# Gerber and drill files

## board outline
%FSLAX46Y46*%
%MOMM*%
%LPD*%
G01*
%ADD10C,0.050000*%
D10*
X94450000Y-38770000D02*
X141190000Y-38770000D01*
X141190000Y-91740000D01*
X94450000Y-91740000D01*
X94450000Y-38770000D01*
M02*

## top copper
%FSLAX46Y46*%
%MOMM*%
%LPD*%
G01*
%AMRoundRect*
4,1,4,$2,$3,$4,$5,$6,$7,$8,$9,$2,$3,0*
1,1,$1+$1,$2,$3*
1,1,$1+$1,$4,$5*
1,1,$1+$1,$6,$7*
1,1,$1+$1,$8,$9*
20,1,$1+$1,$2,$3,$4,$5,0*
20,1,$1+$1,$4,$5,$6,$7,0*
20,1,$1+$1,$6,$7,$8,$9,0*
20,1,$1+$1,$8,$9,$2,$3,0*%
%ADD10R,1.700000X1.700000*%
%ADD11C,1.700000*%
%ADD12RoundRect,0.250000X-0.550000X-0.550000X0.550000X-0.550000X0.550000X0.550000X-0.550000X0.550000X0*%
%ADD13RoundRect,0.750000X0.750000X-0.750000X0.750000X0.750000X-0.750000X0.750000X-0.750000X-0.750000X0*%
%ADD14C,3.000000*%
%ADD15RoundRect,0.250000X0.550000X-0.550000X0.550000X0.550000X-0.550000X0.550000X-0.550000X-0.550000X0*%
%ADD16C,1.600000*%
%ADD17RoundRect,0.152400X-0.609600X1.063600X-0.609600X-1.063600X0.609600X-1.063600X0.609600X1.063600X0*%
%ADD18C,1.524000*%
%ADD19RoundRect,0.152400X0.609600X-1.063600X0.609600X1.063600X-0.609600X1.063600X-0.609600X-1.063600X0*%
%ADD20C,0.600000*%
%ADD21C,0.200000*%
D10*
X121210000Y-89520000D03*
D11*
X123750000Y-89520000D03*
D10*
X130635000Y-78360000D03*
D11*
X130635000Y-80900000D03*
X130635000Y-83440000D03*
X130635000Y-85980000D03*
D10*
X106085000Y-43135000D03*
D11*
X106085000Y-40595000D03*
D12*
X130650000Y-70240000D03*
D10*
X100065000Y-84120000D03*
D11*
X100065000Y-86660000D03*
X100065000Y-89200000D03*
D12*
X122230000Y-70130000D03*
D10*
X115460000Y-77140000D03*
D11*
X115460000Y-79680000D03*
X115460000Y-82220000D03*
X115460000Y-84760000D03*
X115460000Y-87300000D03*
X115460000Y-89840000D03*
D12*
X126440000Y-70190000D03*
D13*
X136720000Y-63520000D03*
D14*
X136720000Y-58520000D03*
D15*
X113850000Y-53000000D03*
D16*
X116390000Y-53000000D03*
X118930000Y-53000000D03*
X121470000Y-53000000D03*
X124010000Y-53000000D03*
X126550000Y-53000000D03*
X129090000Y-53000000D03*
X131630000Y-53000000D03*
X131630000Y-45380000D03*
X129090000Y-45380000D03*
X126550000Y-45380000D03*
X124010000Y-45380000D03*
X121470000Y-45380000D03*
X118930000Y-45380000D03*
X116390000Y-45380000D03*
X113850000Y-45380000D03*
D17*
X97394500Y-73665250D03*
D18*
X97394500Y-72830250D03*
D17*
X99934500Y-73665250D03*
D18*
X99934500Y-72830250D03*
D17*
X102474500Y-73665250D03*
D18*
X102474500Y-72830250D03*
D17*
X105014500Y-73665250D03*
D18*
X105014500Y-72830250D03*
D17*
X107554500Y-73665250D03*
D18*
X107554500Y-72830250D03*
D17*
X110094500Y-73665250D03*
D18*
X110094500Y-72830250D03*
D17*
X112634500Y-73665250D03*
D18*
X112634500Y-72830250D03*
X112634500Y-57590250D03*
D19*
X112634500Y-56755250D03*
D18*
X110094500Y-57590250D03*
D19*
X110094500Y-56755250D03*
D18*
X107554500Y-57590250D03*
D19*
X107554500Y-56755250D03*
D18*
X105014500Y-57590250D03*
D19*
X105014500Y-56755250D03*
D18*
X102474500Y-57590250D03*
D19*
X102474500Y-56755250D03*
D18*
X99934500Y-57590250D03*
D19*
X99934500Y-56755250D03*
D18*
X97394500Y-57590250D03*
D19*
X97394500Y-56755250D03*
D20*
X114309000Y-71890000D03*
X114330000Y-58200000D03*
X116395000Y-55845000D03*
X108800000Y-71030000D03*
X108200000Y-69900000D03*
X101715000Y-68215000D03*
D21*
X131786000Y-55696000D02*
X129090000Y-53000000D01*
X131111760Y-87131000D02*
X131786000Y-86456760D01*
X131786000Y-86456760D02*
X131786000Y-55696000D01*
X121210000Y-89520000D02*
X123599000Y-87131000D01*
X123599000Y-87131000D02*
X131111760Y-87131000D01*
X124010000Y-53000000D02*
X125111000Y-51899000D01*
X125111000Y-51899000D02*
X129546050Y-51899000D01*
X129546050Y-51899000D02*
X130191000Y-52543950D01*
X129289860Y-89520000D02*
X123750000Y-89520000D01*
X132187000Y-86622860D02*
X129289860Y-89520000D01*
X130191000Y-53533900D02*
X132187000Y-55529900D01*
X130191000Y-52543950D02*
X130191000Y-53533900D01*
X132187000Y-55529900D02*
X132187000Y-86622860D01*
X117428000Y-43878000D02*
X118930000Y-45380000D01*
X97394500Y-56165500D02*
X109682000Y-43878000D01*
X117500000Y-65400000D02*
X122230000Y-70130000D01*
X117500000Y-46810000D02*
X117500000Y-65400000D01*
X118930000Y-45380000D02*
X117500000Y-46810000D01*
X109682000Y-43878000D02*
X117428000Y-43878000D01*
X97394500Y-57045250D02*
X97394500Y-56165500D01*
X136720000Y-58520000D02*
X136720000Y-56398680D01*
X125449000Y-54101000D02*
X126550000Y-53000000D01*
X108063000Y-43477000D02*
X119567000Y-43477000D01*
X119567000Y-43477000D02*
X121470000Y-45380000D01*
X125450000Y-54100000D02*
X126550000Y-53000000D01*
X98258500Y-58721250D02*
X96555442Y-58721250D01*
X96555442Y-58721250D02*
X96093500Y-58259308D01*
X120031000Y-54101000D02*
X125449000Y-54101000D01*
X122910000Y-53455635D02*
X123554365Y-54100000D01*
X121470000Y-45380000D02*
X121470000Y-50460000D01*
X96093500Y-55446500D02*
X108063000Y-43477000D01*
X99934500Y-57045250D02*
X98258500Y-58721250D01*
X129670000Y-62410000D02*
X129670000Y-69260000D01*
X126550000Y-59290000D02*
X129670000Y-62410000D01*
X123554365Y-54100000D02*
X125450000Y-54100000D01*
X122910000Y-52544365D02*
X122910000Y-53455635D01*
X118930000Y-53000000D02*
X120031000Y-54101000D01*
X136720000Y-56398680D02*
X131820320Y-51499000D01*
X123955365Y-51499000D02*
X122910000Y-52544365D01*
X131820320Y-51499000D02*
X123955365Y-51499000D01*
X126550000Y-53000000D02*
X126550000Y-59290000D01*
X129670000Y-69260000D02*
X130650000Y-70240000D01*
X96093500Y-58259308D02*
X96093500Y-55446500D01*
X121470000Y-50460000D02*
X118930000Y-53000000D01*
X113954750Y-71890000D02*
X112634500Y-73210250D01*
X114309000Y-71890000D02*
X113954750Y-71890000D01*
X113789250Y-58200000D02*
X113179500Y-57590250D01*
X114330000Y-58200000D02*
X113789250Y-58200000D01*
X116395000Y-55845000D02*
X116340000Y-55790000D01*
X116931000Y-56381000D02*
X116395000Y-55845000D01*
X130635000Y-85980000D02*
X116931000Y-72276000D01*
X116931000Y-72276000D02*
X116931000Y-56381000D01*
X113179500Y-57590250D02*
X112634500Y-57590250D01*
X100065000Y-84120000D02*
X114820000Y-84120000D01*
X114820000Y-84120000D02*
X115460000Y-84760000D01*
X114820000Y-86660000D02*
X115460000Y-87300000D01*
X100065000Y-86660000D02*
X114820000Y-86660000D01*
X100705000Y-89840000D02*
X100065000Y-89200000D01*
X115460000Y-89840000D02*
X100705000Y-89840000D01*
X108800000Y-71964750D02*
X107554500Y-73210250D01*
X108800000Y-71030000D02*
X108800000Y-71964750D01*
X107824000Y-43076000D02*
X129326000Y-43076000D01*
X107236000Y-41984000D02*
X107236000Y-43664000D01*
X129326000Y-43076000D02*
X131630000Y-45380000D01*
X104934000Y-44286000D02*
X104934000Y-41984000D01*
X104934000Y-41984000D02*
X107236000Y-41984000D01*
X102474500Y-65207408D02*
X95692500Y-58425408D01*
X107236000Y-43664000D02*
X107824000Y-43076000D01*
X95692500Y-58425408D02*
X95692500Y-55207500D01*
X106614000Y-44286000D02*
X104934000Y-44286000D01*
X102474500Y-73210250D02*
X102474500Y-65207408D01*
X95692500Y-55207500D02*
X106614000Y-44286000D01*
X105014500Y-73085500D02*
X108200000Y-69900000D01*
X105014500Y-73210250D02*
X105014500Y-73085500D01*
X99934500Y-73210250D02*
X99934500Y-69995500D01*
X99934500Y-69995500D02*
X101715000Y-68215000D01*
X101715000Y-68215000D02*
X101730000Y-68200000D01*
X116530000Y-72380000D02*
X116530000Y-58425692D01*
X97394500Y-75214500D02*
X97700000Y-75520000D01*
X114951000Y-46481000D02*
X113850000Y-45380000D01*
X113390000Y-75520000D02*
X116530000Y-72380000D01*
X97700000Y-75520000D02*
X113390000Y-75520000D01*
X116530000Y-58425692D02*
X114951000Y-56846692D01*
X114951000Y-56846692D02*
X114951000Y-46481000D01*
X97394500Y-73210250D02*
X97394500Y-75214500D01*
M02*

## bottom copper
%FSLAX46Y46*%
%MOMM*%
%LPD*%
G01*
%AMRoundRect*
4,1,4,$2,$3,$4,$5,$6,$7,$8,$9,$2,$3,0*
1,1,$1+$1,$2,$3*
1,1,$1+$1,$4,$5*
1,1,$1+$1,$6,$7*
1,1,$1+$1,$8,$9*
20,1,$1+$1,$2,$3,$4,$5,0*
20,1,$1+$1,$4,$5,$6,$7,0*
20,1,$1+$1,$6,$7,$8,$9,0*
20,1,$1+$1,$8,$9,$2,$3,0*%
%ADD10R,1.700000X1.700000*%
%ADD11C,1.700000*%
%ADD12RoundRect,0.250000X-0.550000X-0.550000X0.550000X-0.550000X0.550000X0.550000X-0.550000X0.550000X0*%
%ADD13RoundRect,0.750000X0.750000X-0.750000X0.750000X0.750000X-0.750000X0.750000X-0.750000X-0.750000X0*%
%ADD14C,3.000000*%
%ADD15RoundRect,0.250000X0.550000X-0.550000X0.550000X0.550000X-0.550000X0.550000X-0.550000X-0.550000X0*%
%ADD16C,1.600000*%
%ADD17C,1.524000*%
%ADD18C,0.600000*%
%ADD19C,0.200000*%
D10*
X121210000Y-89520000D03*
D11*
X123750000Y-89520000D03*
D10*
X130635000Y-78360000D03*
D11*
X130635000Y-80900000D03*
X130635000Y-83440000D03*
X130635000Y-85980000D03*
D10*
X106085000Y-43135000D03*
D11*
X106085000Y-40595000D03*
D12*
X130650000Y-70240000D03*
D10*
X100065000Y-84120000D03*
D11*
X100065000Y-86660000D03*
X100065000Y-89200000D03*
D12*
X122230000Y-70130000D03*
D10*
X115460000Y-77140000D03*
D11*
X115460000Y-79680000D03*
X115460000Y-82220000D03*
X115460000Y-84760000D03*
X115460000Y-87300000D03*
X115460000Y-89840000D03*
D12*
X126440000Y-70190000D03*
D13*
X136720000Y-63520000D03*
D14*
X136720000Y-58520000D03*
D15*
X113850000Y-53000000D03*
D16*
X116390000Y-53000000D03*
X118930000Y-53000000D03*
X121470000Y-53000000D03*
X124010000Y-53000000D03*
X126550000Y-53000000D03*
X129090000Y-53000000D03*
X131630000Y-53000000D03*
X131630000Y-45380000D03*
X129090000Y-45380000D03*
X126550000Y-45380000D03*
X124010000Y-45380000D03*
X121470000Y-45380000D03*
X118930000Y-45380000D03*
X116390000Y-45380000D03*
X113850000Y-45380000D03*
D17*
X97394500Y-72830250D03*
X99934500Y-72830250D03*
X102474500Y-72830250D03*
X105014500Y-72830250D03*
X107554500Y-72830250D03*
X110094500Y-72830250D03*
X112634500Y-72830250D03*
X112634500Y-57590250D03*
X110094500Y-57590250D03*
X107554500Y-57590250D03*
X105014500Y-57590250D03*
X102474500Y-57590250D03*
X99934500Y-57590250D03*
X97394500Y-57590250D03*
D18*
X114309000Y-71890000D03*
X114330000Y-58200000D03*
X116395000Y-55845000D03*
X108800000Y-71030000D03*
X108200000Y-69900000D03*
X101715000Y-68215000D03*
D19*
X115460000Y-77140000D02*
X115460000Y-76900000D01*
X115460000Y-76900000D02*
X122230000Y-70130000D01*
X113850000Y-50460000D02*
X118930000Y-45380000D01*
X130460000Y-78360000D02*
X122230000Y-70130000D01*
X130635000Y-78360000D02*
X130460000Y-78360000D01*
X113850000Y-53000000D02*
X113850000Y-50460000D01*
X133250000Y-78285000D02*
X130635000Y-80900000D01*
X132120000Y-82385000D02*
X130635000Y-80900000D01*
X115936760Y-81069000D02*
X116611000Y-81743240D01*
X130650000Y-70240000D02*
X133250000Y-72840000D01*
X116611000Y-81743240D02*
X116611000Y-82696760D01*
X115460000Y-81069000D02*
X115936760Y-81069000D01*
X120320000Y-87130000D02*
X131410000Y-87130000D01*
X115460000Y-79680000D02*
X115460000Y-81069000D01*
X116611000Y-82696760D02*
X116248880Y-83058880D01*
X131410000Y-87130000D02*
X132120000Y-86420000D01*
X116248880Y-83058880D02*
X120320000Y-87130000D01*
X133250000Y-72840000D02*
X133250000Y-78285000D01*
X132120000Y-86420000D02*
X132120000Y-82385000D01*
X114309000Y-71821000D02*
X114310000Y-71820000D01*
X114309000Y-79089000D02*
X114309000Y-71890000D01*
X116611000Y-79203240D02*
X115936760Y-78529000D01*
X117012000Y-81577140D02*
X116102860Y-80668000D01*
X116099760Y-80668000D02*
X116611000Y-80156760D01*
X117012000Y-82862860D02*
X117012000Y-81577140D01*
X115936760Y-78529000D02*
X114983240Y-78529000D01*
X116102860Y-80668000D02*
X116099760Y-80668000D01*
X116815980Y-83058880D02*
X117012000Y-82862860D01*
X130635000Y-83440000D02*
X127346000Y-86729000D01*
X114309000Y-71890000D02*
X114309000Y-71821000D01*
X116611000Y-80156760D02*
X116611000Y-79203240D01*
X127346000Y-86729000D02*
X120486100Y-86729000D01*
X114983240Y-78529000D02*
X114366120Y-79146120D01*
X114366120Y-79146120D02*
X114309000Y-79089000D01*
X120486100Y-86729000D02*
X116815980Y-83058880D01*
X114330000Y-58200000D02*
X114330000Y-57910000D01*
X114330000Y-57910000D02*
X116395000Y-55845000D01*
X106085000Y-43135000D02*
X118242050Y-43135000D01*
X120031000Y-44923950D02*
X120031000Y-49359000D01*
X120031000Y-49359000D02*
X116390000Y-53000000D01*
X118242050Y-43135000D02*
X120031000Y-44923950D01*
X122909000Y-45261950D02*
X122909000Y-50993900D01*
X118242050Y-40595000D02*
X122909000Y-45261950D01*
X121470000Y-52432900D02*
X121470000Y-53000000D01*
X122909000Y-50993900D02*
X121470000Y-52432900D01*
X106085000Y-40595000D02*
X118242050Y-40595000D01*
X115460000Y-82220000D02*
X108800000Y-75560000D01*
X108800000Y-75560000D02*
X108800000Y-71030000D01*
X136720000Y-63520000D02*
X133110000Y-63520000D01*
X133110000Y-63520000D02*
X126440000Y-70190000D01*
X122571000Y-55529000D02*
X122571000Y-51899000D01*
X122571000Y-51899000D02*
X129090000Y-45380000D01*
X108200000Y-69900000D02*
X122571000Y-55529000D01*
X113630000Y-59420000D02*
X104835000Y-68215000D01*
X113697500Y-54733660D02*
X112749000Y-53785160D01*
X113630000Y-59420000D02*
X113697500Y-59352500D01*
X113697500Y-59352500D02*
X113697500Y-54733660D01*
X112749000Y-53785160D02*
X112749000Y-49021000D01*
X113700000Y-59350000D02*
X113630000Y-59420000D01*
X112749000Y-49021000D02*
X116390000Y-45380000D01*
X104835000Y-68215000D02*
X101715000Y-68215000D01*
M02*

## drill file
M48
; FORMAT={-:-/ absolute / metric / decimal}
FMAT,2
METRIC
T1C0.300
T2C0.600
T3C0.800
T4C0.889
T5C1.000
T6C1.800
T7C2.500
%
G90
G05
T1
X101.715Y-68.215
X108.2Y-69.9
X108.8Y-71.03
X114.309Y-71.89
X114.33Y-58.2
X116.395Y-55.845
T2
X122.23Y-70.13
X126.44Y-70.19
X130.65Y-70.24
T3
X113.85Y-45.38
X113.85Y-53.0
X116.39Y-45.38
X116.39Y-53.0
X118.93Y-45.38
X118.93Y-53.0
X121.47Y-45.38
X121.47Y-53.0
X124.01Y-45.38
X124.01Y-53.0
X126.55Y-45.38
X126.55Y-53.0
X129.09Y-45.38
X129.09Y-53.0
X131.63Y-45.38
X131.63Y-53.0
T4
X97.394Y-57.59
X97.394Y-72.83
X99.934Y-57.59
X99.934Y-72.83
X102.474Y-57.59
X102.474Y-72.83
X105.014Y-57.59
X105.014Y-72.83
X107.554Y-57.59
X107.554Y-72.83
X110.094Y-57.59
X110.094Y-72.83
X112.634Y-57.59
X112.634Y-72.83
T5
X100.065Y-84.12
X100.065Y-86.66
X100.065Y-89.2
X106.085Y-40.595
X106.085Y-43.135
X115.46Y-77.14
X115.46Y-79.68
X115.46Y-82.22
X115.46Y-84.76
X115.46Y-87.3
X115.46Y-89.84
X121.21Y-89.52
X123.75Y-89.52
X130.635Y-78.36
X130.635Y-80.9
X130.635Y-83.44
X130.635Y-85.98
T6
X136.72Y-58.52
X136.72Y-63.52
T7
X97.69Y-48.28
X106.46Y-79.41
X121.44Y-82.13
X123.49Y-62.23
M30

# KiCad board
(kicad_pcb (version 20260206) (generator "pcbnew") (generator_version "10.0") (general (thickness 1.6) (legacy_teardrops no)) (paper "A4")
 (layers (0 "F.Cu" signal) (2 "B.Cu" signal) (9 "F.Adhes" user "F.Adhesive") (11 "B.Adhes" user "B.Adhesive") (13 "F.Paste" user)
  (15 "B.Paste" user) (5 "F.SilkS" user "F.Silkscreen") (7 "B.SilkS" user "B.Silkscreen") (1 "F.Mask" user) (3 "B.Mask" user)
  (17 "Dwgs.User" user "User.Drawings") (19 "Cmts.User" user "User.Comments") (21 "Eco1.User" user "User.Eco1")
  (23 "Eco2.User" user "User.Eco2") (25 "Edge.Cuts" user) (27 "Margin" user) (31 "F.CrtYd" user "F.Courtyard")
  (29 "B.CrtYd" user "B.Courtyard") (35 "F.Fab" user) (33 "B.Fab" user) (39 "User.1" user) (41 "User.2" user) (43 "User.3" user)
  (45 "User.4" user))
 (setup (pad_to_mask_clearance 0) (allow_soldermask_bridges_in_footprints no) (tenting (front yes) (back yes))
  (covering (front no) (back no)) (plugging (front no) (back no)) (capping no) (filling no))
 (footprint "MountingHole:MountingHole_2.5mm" (layer "F.Cu") (at 123.49 62.23)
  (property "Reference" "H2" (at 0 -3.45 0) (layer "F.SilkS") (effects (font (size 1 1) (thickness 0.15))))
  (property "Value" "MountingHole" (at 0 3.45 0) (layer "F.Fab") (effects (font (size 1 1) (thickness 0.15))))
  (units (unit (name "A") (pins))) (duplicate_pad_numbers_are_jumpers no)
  (pad "" np_thru_hole circle (at 0 0) (size 2.5 2.5) (drill 2.5) (layers "*.Cu" "*.Mask")))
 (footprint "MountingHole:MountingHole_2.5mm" (layer "F.Cu") (at 106.46 79.41)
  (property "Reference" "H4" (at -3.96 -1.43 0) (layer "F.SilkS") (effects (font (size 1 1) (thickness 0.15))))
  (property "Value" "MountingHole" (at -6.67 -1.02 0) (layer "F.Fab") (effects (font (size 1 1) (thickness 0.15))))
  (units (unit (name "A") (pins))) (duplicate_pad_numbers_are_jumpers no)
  (pad "" np_thru_hole circle (at 0 0) (size 2.5 2.5) (drill 2.5) (layers "*.Cu" "*.Mask")))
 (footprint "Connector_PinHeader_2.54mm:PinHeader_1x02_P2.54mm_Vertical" (layer "F.Cu") (at 121.21 89.52 90)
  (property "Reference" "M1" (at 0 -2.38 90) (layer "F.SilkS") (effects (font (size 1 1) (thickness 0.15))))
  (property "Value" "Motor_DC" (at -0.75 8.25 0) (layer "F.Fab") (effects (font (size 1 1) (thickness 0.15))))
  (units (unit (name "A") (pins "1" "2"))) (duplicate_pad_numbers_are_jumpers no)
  (pad "1" thru_hole rect (at 0 0 90) (size 1.7 1.7) (drill 1) (layers "*.Cu" "*.Mask") (remove_unused_layers no) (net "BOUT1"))
  (pad "2" thru_hole circle (at 0 2.54 90) (size 1.7 1.7) (drill 1) (layers "*.Cu" "*.Mask") (remove_unused_layers no) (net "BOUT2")))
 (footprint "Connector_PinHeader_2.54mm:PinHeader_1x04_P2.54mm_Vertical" (layer "F.Cu") (at 130.635 78.36)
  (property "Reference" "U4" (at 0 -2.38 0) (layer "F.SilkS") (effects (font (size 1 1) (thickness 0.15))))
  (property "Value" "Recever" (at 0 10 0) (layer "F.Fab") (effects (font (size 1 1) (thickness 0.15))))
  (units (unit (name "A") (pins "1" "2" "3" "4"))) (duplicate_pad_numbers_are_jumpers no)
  (pad "1" thru_hole rect (at 0 0) (size 1.7 1.7) (drill 1) (layers "*.Cu" "*.Mask") (remove_unused_layers no) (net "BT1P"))
  (pad "2" thru_hole circle (at 0 2.54) (size 1.7 1.7) (drill 1) (layers "*.Cu" "*.Mask") (remove_unused_layers no) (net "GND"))
  (pad "3" thru_hole circle (at 0 5.08) (size 1.7 1.7) (drill 1) (layers "*.Cu" "*.Mask") (remove_unused_layers no)
   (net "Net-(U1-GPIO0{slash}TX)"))
  (pad "4" thru_hole circle (at 0 7.62) (size 1.7 1.7) (drill 1) (layers "*.Cu" "*.Mask") (remove_unused_layers no)
   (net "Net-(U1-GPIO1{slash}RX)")))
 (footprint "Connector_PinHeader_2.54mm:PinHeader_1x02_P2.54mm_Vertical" (layer "F.Cu") (at 106.085 43.135 180)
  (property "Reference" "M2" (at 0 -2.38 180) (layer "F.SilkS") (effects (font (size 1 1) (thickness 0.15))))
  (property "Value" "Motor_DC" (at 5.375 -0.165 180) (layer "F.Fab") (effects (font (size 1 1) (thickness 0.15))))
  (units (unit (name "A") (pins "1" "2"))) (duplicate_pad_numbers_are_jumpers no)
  (pad "1" thru_hole rect (at 0 0 180) (size 1.7 1.7) (drill 1) (layers "*.Cu" "*.Mask") (remove_unused_layers no) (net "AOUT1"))
  (pad "2" thru_hole circle (at 0 2.54 180) (size 1.7 1.7) (drill 1) (layers "*.Cu" "*.Mask") (remove_unused_layers no) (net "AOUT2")))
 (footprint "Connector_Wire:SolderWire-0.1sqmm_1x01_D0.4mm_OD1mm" (layer "F.Cu") (at 130.65 70.24)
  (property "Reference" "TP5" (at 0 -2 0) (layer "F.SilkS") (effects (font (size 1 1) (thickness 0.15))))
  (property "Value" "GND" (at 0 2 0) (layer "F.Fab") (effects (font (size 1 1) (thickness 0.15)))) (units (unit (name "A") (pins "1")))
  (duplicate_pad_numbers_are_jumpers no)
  (pad "1" thru_hole roundrect (at 0 0) (size 1.6 1.6) (drill 0.6) (layers "*.Cu" "*.Mask") (remove_unused_layers no)
   (roundrect_rratio 0.15625) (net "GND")))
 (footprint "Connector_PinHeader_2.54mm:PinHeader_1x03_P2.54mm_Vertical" (layer "F.Cu") (at 100.065 84.12)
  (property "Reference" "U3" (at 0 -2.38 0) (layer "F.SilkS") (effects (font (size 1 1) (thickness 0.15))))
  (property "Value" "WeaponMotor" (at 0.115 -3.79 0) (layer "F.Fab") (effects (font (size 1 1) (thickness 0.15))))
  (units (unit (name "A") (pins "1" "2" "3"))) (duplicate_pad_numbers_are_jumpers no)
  (pad "1" thru_hole rect (at 0 0) (size 1.7 1.7) (drill 1) (layers "*.Cu" "*.Mask") (remove_unused_layers no) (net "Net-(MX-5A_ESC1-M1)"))
  (pad "2" thru_hole circle (at 0 2.54) (size 1.7 1.7) (drill 1) (layers "*.Cu" "*.Mask") (remove_unused_layers no)
   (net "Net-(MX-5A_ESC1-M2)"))
  (pad "3" thru_hole circle (at 0 5.08) (size 1.7 1.7) (drill 1) (layers "*.Cu" "*.Mask") (remove_unused_layers no)
   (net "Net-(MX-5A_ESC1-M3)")))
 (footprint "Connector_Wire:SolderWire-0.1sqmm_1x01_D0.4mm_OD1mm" (layer "F.Cu") (at 122.23 70.13)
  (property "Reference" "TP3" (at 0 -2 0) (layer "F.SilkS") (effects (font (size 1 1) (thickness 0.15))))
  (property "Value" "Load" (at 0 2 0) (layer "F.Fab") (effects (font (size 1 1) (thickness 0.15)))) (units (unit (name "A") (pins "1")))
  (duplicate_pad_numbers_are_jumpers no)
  (pad "1" thru_hole roundrect (at 0 0) (size 1.6 1.6) (drill 0.6) (layers "*.Cu" "*.Mask") (remove_unused_layers no)
   (roundrect_rratio 0.15625) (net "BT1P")))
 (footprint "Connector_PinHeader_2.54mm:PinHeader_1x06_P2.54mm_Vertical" (layer "F.Cu") (at 115.46 77.14)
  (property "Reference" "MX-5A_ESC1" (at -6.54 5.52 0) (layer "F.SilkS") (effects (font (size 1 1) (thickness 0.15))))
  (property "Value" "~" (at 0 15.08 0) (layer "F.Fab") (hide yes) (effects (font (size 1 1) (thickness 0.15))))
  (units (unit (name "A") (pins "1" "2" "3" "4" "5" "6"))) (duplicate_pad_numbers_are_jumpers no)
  (pad "1" thru_hole rect (at 0 0) (size 1.7 1.7) (drill 1) (layers "*.Cu" "*.Mask") (remove_unused_layers no) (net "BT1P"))
  (pad "2" thru_hole circle (at 0 2.54) (size 1.7 1.7) (drill 1) (layers "*.Cu" "*.Mask") (remove_unused_layers no) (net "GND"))
  (pad "3" thru_hole circle (at 0 5.08) (size 1.7 1.7) (drill 1) (layers "*.Cu" "*.Mask") (remove_unused_layers no)
   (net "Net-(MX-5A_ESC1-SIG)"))
  (pad "4" thru_hole circle (at 0 7.62) (size 1.7 1.7) (drill 1) (layers "*.Cu" "*.Mask") (remove_unused_layers no)
   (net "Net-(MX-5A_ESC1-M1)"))
  (pad "5" thru_hole circle (at 0 10.16) (size 1.7 1.7) (drill 1) (layers "*.Cu" "*.Mask") (remove_unused_layers no)
   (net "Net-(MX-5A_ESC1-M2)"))
  (pad "6" thru_hole circle (at 0 12.7) (size 1.7 1.7) (drill 1) (layers "*.Cu" "*.Mask") (remove_unused_layers no)
   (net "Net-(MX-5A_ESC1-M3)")))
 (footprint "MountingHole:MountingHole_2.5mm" (layer "F.Cu") (at 121.44 82.13)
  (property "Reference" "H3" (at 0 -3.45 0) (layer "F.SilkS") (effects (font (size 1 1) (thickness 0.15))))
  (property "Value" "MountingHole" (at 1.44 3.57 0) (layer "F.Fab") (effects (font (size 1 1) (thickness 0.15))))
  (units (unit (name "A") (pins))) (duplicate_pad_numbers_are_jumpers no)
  (pad "" np_thru_hole circle (at 0 0) (size 2.5 2.5) (drill 2.5) (layers "*.Cu" "*.Mask")))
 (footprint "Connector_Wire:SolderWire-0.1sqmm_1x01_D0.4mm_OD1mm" (layer "F.Cu") (at 126.44 70.19)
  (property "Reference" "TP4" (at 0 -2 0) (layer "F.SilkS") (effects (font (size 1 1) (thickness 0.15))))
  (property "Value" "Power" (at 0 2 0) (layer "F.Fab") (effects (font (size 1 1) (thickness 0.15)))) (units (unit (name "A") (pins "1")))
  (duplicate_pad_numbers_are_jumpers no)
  (pad "1" thru_hole roundrect (at 0 0) (size 1.6 1.6) (drill 0.6) (layers "*.Cu" "*.Mask") (remove_unused_layers no)
   (roundrect_rratio 0.15625) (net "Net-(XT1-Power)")))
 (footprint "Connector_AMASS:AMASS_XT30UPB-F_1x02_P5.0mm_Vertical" (layer "F.Cu") (at 136.72 63.52 90)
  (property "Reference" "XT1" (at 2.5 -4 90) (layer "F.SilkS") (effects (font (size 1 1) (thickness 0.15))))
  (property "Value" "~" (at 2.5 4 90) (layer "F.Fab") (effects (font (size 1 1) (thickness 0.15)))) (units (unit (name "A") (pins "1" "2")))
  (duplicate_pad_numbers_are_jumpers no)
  (pad "1" thru_hole roundrect (at 0 0 90) (size 3 3) (drill 1.8) (layers "*.Cu" "*.Mask") (remove_unused_layers no) (roundrect_rratio 0.25)
   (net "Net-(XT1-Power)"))
  (pad "2" thru_hole circle (at 5 0 90) (size 3 3) (drill 1.8) (layers "*.Cu" "*.Mask") (remove_unused_layers no) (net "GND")))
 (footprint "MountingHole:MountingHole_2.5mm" (layer "F.Cu") (at 97.69 48.28)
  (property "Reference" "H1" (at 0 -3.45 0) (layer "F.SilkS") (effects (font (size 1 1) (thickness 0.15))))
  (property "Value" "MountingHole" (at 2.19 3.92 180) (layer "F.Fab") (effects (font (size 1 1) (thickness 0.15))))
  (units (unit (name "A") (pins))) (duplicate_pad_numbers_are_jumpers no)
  (pad "" np_thru_hole circle (at 0 0) (size 2.5 2.5) (drill 2.5) (layers "*.Cu" "*.Mask")))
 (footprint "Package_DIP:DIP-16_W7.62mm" (layer "F.Cu") (at 113.85 53 90)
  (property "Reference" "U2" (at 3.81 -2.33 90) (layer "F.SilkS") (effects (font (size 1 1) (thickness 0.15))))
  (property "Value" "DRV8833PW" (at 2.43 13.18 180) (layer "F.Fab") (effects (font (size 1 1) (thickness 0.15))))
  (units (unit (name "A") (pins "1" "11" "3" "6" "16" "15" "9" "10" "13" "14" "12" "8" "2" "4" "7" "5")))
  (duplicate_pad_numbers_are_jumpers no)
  (pad "1" thru_hole roundrect (at 0 0 90) (size 1.6 1.6) (drill 0.8) (layers "*.Cu" "*.Mask") (remove_unused_layers no)
   (roundrect_rratio 0.15625) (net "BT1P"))
  (pad "2" thru_hole circle (at 0 2.54 90) (size 1.6 1.6) (drill 0.8) (layers "*.Cu" "*.Mask") (remove_unused_layers no) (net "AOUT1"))
  (pad "3" thru_hole circle (at 0 5.08 90) (size 1.6 1.6) (drill 0.8) (layers "*.Cu" "*.Mask") (remove_unused_layers no) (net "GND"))
  (pad "4" thru_hole circle (at 0 7.62 90) (size 1.6 1.6) (drill 0.8) (layers "*.Cu" "*.Mask") (remove_unused_layers no) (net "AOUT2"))
  (pad "5" thru_hole circle (at 0 10.16 90) (size 1.6 1.6) (drill 0.8) (layers "*.Cu" "*.Mask") (remove_unused_layers no) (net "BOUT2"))
  (pad "6" thru_hole circle (at 0 12.7 90) (size 1.6 1.6) (drill 0.8) (layers "*.Cu" "*.Mask") (remove_unused_layers no) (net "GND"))
  (pad "7" thru_hole circle (at 0 15.24 90) (size 1.6 1.6) (drill 0.8) (layers "*.Cu" "*.Mask") (remove_unused_layers no) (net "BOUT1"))
  (pad "8" thru_hole circle (at 0 17.78 90) (size 1.6 1.6) (drill 0.8) (layers "*.Cu" "*.Mask") (remove_unused_layers no)
   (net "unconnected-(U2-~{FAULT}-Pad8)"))
  (pad "9" thru_hole circle (at 7.62 17.78 90) (size 1.6 1.6) (drill 0.8) (layers "*.Cu" "*.Mask") (remove_unused_layers no) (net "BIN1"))
  (pad "10" thru_hole circle (at 7.62 15.24 90) (size 1.6 1.6) (drill 0.8) (layers "*.Cu" "*.Mask") (remove_unused_layers no) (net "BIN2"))
  (pad "11" thru_hole circle (at 7.62 12.7 90) (size 1.6 1.6) (drill 0.8) (layers "*.Cu" "*.Mask") (remove_unused_layers no)
   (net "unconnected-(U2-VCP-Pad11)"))
  (pad "12" thru_hole circle (at 7.62 10.16 90) (size 1.6 1.6) (drill 0.8) (layers "*.Cu" "*.Mask") (remove_unused_layers no)
   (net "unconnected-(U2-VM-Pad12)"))
  (pad "13" thru_hole circle (at 7.62 7.62 90) (size 1.6 1.6) (drill 0.8) (layers "*.Cu" "*.Mask") (remove_unused_layers no) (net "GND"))
  (pad "14" thru_hole circle (at 7.62 5.08 90) (size 1.6 1.6) (drill 0.8) (layers "*.Cu" "*.Mask") (remove_unused_layers no) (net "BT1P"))
  (pad "15" thru_hole circle (at 7.62 2.54 90) (size 1.6 1.6) (drill 0.8) (layers "*.Cu" "*.Mask") (remove_unused_layers no) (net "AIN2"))
  (pad "16" thru_hole circle (at 7.62 0 90) (size 1.6 1.6) (drill 0.8) (layers "*.Cu" "*.Mask") (remove_unused_layers no) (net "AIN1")))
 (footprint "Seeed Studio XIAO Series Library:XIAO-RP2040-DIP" (layer "F.Cu") (at 105.0145 65.21025 90)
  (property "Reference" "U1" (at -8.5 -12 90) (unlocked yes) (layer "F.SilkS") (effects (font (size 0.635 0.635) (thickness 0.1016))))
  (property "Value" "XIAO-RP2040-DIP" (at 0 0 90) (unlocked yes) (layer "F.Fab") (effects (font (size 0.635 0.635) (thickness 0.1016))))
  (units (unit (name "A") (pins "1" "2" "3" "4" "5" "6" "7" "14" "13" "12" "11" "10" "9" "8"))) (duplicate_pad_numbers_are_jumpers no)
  (pad "1" smd roundrect (at -8.455 -7.62 270) (size 2.432 1.524) (layers "F.Cu" "F.Mask") (roundrect_rratio 0.1) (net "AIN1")
   (thermal_bridge_angle 45))
  (pad "1" thru_hole circle (at -7.62 -7.62 270) (size 1.524 1.524) (drill 0.889) (layers "*.Cu" "*.Mask") (remove_unused_layers no)
   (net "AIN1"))
  (pad "2" smd roundrect (at -8.455 -5.08 270) (size 2.432 1.524) (layers "F.Cu" "F.Mask") (roundrect_rratio 0.1) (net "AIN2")
   (thermal_bridge_angle 45))
  (pad "2" thru_hole circle (at -7.62 -5.08 270) (size 1.524 1.524) (drill 0.889) (layers "*.Cu" "*.Mask") (remove_unused_layers no)
   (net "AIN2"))
  (pad "3" smd roundrect (at -8.455 -2.54 270) (size 2.432 1.524) (layers "F.Cu" "F.Mask") (roundrect_rratio 0.1) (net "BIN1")
   (thermal_bridge_angle 45))
  (pad "3" thru_hole circle (at -7.62 -2.54 270) (size 1.524 1.524) (drill 0.889) (layers "*.Cu" "*.Mask") (remove_unused_layers no)
   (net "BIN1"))
  (pad "4" smd roundrect (at -8.455 0 270) (size 2.432 1.524) (layers "F.Cu" "F.Mask") (roundrect_rratio 0.1) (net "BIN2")
   (thermal_bridge_angle 45))
  (pad "4" thru_hole circle (at -7.62 0 270) (size 1.524 1.524) (drill 0.889) (layers "*.Cu" "*.Mask") (remove_unused_layers no)
   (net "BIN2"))
  (pad "5" smd roundrect (at -8.455 2.54 270) (size 2.432 1.524) (layers "F.Cu" "F.Mask") (roundrect_rratio 0.1)
   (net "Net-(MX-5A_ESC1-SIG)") (thermal_bridge_angle 45))
  (pad "5" thru_hole circle (at -7.62 2.54 270) (size 1.524 1.524) (drill 0.889) (layers "*.Cu" "*.Mask") (remove_unused_layers no)
   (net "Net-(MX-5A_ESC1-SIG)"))
  (pad "6" smd roundrect (at -8.455 5.08 270) (size 2.432 1.524) (layers "F.Cu" "F.Mask") (roundrect_rratio 0.1)
   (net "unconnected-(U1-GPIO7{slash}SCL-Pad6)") (thermal_bridge_angle 45))
  (pad "6" thru_hole circle (at -7.62 5.08 270) (size 1.524 1.524) (drill 0.889) (layers "*.Cu" "*.Mask") (remove_unused_layers no)
   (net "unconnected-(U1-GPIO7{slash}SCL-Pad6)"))
  (pad "7" smd roundrect (at -8.455 7.62 270) (size 2.432 1.524) (layers "F.Cu" "F.Mask") (roundrect_rratio 0.1)
   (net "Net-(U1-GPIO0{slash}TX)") (thermal_bridge_angle 45))
  (pad "7" thru_hole circle (at -7.62 7.62 270) (size 1.524 1.524) (drill 0.889) (layers "*.Cu" "*.Mask") (remove_unused_layers no)
   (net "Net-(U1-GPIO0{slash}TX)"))
  (pad "8" thru_hole circle (at 7.62 7.62 90) (size 1.524 1.524) (drill 0.889) (layers "*.Cu" "*.Mask") (remove_unused_layers no)
   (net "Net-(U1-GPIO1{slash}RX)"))
  (pad "8" smd roundrect (at 8.455 7.62 90) (size 2.432 1.524) (layers "F.Cu" "F.Mask") (roundrect_rratio 0.1)
   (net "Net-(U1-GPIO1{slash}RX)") (thermal_bridge_angle 45))
  (pad "9" thru_hole circle (at 7.62 5.08 90) (size 1.524 1.524) (drill 0.889) (layers "*.Cu" "*.Mask") (remove_unused_layers no)
   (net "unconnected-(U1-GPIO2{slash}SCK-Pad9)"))
  (pad "9" smd roundrect (at 8.455 5.08 90) (size 2.432 1.524) (layers "F.Cu" "F.Mask") (roundrect_rratio 0.1)
   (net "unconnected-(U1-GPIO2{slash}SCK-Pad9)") (thermal_bridge_angle 45))
  (pad "10" thru_hole circle (at 7.62 2.54 90) (size 1.524 1.524) (drill 0.889) (layers "*.Cu" "*.Mask") (remove_unused_layers no)
   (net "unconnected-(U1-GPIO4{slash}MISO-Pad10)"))
  (pad "10" smd roundrect (at 8.455 2.54 90) (size 2.432 1.524) (layers "F.Cu" "F.Mask") (roundrect_rratio 0.1)
   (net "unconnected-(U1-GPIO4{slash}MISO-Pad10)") (thermal_bridge_angle 45))
  (pad "11" thru_hole circle (at 7.62 0 90) (size 1.524 1.524) (drill 0.889) (layers "*.Cu" "*.Mask") (remove_unused_layers no)
   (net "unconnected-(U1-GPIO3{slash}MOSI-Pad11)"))
  (pad "11" smd roundrect (at 8.455 0 90) (size 2.432 1.524) (layers "F.Cu" "F.Mask") (roundrect_rratio 0.1)
   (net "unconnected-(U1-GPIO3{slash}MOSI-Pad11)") (thermal_bridge_angle 45))
  (pad "12" thru_hole circle (at 7.62 -2.54 90) (size 1.524 1.524) (drill 0.889) (layers "*.Cu" "*.Mask") (remove_unused_layers no)
   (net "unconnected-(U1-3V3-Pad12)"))
  (pad "12" smd roundrect (at 8.455 -2.54 90) (size 2.432 1.524) (layers "F.Cu" "F.Mask") (roundrect_rratio 0.1)
   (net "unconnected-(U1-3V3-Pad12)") (thermal_bridge_angle 45))
  (pad "13" thru_hole circle (at 7.62 -5.08 90) (size 1.524 1.524) (drill 0.889) (layers "*.Cu" "*.Mask") (remove_unused_layers no)
   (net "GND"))
  (pad "13" smd roundrect (at 8.455 -5.08 90) (size 2.432 1.524) (layers "F.Cu" "F.Mask") (roundrect_rratio 0.1) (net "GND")
   (thermal_bridge_angle 45))
  (pad "14" thru_hole circle (at 7.62 -7.62 90) (size 1.524 1.524) (drill 0.889) (layers "*.Cu" "*.Mask") (remove_unused_layers no)
   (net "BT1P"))
  (pad "14" smd roundrect (at 8.455 -7.62 90) (size 2.432 1.524) (layers "F.Cu" "F.Mask") (roundrect_rratio 0.1) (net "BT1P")
   (thermal_bridge_angle 45)))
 (gr_rect (start 94.45 38.77) (end 141.19 91.74) (stroke (width 0.05) (type default)) (fill no) (layer "Edge.Cuts"))
 (segment (start 131.786 55.696) (end 129.09 53) (width 0.2) (layer "F.Cu") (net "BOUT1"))
 (segment (start 131.11176 87.131) (end 131.786 86.45676) (width 0.2) (layer "F.Cu") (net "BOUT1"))
 (segment (start 131.786 86.45676) (end 131.786 55.696) (width 0.2) (layer "F.Cu") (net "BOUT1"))
 (segment (start 121.21 89.52) (end 123.599 87.131) (width 0.2) (layer "F.Cu") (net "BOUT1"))
 (segment (start 123.599 87.131) (end 131.11176 87.131) (width 0.2) (layer "F.Cu") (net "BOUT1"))
 (segment (start 124.01 53) (end 125.111 51.899) (width 0.2) (layer "F.Cu") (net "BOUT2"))
 (segment (start 125.111 51.899) (end 129.54605 51.899) (width 0.2) (layer "F.Cu") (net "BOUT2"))
 (segment (start 129.54605 51.899) (end 130.191 52.54395) (width 0.2) (layer "F.Cu") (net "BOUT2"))
 (segment (start 129.28986 89.52) (end 123.75 89.52) (width 0.2) (layer "F.Cu") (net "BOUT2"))
 (segment (start 132.187 86.62286) (end 129.28986 89.52) (width 0.2) (layer "F.Cu") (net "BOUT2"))
 (segment (start 130.191 53.5339) (end 132.187 55.5299) (width 0.2) (layer "F.Cu") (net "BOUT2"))
 (segment (start 130.191 52.54395) (end 130.191 53.5339) (width 0.2) (layer "F.Cu") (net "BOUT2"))
 (segment (start 132.187 55.5299) (end 132.187 86.62286) (width 0.2) (layer "F.Cu") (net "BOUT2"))
 (segment (start 117.428 43.878) (end 118.93 45.38) (width 0.2) (layer "F.Cu") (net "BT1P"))
 (segment (start 97.3945 56.1655) (end 109.682 43.878) (width 0.2) (layer "F.Cu") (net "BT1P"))
 (segment (start 117.5 65.4) (end 122.23 70.13) (width 0.2) (layer "F.Cu") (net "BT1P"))
 (segment (start 117.5 46.81) (end 117.5 65.4) (width 0.2) (layer "F.Cu") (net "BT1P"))
 (segment (start 118.93 45.38) (end 117.5 46.81) (width 0.2) (layer "F.Cu") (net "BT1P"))
 (segment (start 109.682 43.878) (end 117.428 43.878) (width 0.2) (layer "F.Cu") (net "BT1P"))
 (segment (start 97.3945 57.04525) (end 97.3945 56.1655) (width 0.2) (layer "F.Cu") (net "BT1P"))
 (segment (start 115.46 77.14) (end 115.46 76.9) (width 0.2) (layer "B.Cu") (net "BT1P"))
 (segment (start 115.46 76.9) (end 122.23 70.13) (width 0.2) (layer "B.Cu") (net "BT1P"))
 (segment (start 113.85 50.46) (end 118.93 45.38) (width 0.2) (layer "B.Cu") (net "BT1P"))
 (segment (start 130.46 78.36) (end 122.23 70.13) (width 0.2) (layer "B.Cu") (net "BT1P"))
 (segment (start 130.635 78.36) (end 130.46 78.36) (width 0.2) (layer "B.Cu") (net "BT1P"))
 (segment (start 113.85 53) (end 113.85 50.46) (width 0.2) (layer "B.Cu") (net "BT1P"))
 (segment (start 136.72 58.52) (end 136.72 56.39868) (width 0.2) (layer "F.Cu") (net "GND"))
 (segment (start 125.449 54.101) (end 126.55 53) (width 0.2) (layer "F.Cu") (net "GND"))
 (segment (start 108.063 43.477) (end 119.567 43.477) (width 0.2) (layer "F.Cu") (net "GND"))
 (segment (start 119.567 43.477) (end 121.47 45.38) (width 0.2) (layer "F.Cu") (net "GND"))
 (segment (start 125.45 54.1) (end 126.55 53) (width 0.2) (layer "F.Cu") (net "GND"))
 (segment (start 98.2585 58.72125) (end 96.555442 58.72125) (width 0.2) (layer "F.Cu") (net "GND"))
 (segment (start 96.555442 58.72125) (end 96.0935 58.259308) (width 0.2) (layer "F.Cu") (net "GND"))
 (segment (start 120.031 54.101) (end 125.449 54.101) (width 0.2) (layer "F.Cu") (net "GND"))
 (segment (start 122.91 53.455635) (end 123.554365 54.1) (width 0.2) (layer "F.Cu") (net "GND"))
 (segment (start 121.47 45.38) (end 121.47 50.46) (width 0.2) (layer "F.Cu") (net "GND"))
 (segment (start 96.0935 55.4465) (end 108.063 43.477) (width 0.2) (layer "F.Cu") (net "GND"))
 (segment (start 99.9345 57.04525) (end 98.2585 58.72125) (width 0.2) (layer "F.Cu") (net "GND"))
 (segment (start 129.67 62.41) (end 129.67 69.26) (width 0.2) (layer "F.Cu") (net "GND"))
 (segment (start 126.55 59.29) (end 129.67 62.41) (width 0.2) (layer "F.Cu") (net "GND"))
 (segment (start 123.554365 54.1) (end 125.45 54.1) (width 0.2) (layer "F.Cu") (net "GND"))
 (segment (start 122.91 52.544365) (end 122.91 53.455635) (width 0.2) (layer "F.Cu") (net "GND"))
 (segment (start 118.93 53) (end 120.031 54.101) (width 0.2) (layer "F.Cu") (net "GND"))
 (segment (start 136.72 56.39868) (end 131.82032 51.499) (width 0.2) (layer "F.Cu") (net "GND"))
 (segment (start 123.955365 51.499) (end 122.91 52.544365) (width 0.2) (layer "F.Cu") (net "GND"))
 (segment (start 131.82032 51.499) (end 123.955365 51.499) (width 0.2) (layer "F.Cu") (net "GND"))
 (segment (start 126.55 53) (end 126.55 59.29) (width 0.2) (layer "F.Cu") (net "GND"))
 (segment (start 129.67 69.26) (end 130.65 70.24) (width 0.2) (layer "F.Cu") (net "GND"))
 (segment (start 96.0935 58.259308) (end 96.0935 55.4465) (width 0.2) (layer "F.Cu") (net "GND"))
 (segment (start 121.47 50.46) (end 118.93 53) (width 0.2) (layer "F.Cu") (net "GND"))
 (segment (start 133.25 78.285) (end 130.635 80.9) (width 0.2) (layer "B.Cu") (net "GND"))
 (segment (start 132.12 82.385) (end 130.635 80.9) (width 0.2) (layer "B.Cu") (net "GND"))
 (segment (start 115.93676 81.069) (end 116.611 81.74324) (width 0.2) (layer "B.Cu") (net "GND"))
 (segment (start 130.65 70.24) (end 133.25 72.84) (width 0.2) (layer "B.Cu") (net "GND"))
 (segment (start 116.611 81.74324) (end 116.611 82.69676) (width 0.2) (layer "B.Cu") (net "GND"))
 (segment (start 115.46 81.069) (end 115.93676 81.069) (width 0.2) (layer "B.Cu") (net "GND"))
 (segment (start 120.32 87.13) (end 131.41 87.13) (width 0.2) (layer "B.Cu") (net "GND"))
 (segment (start 115.46 79.68) (end 115.46 81.069) (width 0.2) (layer "B.Cu") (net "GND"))
 (segment (start 116.611 82.69676) (end 116.24888 83.05888) (width 0.2) (layer "B.Cu") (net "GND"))
 (segment (start 131.41 87.13) (end 132.12 86.42) (width 0.2) (layer "B.Cu") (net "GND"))
 (segment (start 116.24888 83.05888) (end 120.32 87.13) (width 0.2) (layer "B.Cu") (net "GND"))
 (segment (start 133.25 72.84) (end 133.25 78.285) (width 0.2) (layer "B.Cu") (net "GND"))
 (segment (start 132.12 86.42) (end 132.12 82.385) (width 0.2) (layer "B.Cu") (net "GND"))
 (segment (start 113.95475 71.89) (end 112.6345 73.21025) (width 0.2) (layer "F.Cu") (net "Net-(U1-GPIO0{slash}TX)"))
 (segment (start 114.309 71.89) (end 113.95475 71.89) (width 0.2) (layer "F.Cu") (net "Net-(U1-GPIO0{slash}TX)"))
 (via (at 114.309 71.89) (size 0.6) (drill 0.3) (layers "F.Cu" "B.Cu") (capping no) (covering (front no) (back no))
  (plugging (front no) (back no)) (filling no) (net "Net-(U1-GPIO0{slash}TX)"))
 (segment (start 114.309 71.821) (end 114.31 71.82) (width 0.2) (layer "B.Cu") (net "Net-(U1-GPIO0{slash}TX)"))
 (segment (start 114.309 79.089) (end 114.309 71.89) (width 0.2) (layer "B.Cu") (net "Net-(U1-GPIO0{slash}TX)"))
 (segment (start 116.611 79.20324) (end 115.93676 78.529) (width 0.2) (layer "B.Cu") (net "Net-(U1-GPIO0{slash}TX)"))
 (segment (start 117.012 81.57714) (end 116.10286 80.668) (width 0.2) (layer "B.Cu") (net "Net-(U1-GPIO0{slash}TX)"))
 (segment (start 116.09976 80.668) (end 116.611 80.15676) (width 0.2) (layer "B.Cu") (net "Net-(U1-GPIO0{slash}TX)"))
 (segment (start 117.012 82.86286) (end 117.012 81.57714) (width 0.2) (layer "B.Cu") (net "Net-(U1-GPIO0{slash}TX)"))
 (segment (start 115.93676 78.529) (end 114.98324 78.529) (width 0.2) (layer "B.Cu") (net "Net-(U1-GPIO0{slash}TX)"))
 (segment (start 116.10286 80.668) (end 116.09976 80.668) (width 0.2) (layer "B.Cu") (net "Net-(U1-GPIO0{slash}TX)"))
 (segment (start 116.81598 83.05888) (end 117.012 82.86286) (width 0.2) (layer "B.Cu") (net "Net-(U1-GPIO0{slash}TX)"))
 (segment (start 130.635 83.44) (end 127.346 86.729) (width 0.2) (layer "B.Cu") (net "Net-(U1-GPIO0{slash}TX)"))
 (segment (start 114.309 71.89) (end 114.309 71.821) (width 0.2) (layer "B.Cu") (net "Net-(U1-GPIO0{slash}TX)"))
 (segment (start 116.611 80.15676) (end 116.611 79.20324) (width 0.2) (layer "B.Cu") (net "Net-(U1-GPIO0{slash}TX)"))
 (segment (start 127.346 86.729) (end 120.4861 86.729) (width 0.2) (layer "B.Cu") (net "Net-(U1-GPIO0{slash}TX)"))
 (segment (start 114.98324 78.529) (end 114.36612 79.14612) (width 0.2) (layer "B.Cu") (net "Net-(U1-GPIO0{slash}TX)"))
 (segment (start 114.36612 79.14612) (end 114.309 79.089) (width 0.2) (layer "B.Cu") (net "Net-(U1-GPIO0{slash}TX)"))
 (segment (start 120.4861 86.729) (end 116.81598 83.05888) (width 0.2) (layer "B.Cu") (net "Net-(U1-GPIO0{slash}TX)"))
 (segment (start 113.78925 58.2) (end 113.1795 57.59025) (width 0.2) (layer "F.Cu") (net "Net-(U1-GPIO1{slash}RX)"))
 (segment (start 114.33 58.2) (end 113.78925 58.2) (width 0.2) (layer "F.Cu") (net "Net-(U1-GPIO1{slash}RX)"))
 (segment (start 116.395 55.845) (end 116.34 55.79) (width 0.2) (layer "F.Cu") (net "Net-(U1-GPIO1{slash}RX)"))
 (segment (start 116.931 56.381) (end 116.395 55.845) (width 0.2) (layer "F.Cu") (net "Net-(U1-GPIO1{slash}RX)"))
 (segment (start 130.635 85.98) (end 116.931 72.276) (width 0.2) (layer "F.Cu") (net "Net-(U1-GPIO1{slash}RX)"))
 (segment (start 116.931 72.276) (end 116.931 56.381) (width 0.2) (layer "F.Cu") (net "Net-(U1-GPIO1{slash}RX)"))
 (segment (start 113.1795 57.59025) (end 112.6345 57.59025) (width 0.2) (layer "F.Cu") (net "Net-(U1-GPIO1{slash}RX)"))
 (via (at 114.33 58.2) (size 0.6) (drill 0.3) (layers "F.Cu" "B.Cu") (capping no) (covering (front no) (back no))
  (plugging (front no) (back no)) (filling no) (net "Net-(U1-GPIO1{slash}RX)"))
 (via (at 116.395 55.845) (size 0.6) (drill 0.3) (layers "F.Cu" "B.Cu") (capping no) (covering (front no) (back no))
  (plugging (front no) (back no)) (filling no) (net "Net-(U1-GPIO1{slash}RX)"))
 (segment (start 114.33 58.2) (end 114.33 57.91) (width 0.2) (layer "B.Cu") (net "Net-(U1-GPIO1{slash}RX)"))
 (segment (start 114.33 57.91) (end 116.395 55.845) (width 0.2) (layer "B.Cu") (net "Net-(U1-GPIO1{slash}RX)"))
 (segment (start 106.085 43.135) (end 118.24205 43.135) (width 0.2) (layer "B.Cu") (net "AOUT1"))
 (segment (start 120.031 44.92395) (end 120.031 49.359) (width 0.2) (layer "B.Cu") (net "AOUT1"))
 (segment (start 120.031 49.359) (end 116.39 53) (width 0.2) (layer "B.Cu") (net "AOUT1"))
 (segment (start 118.24205 43.135) (end 120.031 44.92395) (width 0.2) (layer "B.Cu") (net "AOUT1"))
 (segment (start 122.909 45.26195) (end 122.909 50.9939) (width 0.2) (layer "B.Cu") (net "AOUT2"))
 (segment (start 118.24205 40.595) (end 122.909 45.26195) (width 0.2) (layer "B.Cu") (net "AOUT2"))
 (segment (start 121.47 52.4329) (end 121.47 53) (width 0.2) (layer "B.Cu") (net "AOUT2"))
 (segment (start 122.909 50.9939) (end 121.47 52.4329) (width 0.2) (layer "B.Cu") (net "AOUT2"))
 (segment (start 106.085 40.595) (end 118.24205 40.595) (width 0.2) (layer "B.Cu") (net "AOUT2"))
 (segment (start 100.065 84.12) (end 114.82 84.12) (width 0.2) (layer "F.Cu") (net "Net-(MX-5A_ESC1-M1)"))
 (segment (start 114.82 84.12) (end 115.46 84.76) (width 0.2) (layer "F.Cu") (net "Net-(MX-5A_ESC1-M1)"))
 (segment (start 114.82 86.66) (end 115.46 87.3) (width 0.2) (layer "F.Cu") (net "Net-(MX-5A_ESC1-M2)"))
 (segment (start 100.065 86.66) (end 114.82 86.66) (width 0.2) (layer "F.Cu") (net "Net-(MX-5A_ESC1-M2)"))
 (segment (start 100.705 89.84) (end 100.065 89.2) (width 0.2) (layer "F.Cu") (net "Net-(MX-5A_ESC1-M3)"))
 (segment (start 115.46 89.84) (end 100.705 89.84) (width 0.2) (layer "F.Cu") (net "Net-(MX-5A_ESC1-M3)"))
 (segment (start 108.8 71.96475) (end 107.5545 73.21025) (width 0.2) (layer "F.Cu") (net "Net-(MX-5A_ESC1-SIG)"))
 (segment (start 108.8 71.03) (end 108.8 71.96475) (width 0.2) (layer "F.Cu") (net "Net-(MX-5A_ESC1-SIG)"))
 (via (at 108.8 71.03) (size 0.6) (drill 0.3) (layers "F.Cu" "B.Cu") (capping no) (covering (front no) (back no))
  (plugging (front no) (back no)) (filling no) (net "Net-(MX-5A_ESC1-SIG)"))
 (segment (start 115.46 82.22) (end 108.8 75.56) (width 0.2) (layer "B.Cu") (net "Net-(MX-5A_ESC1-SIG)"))
 (segment (start 108.8 75.56) (end 108.8 71.03) (width 0.2) (layer "B.Cu") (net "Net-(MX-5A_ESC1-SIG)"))
 (segment (start 136.72 63.52) (end 133.11 63.52) (width 0.2) (layer "B.Cu") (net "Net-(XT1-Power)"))
 (segment (start 133.11 63.52) (end 126.44 70.19) (width 0.2) (layer "B.Cu") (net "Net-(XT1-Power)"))
 (segment (start 107.824 43.076) (end 129.326 43.076) (width 0.2) (layer "F.Cu") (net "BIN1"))
 (segment (start 107.236 41.984) (end 107.236 43.664) (width 0.2) (layer "F.Cu") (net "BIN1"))
 (segment (start 129.326 43.076) (end 131.63 45.38) (width 0.2) (layer "F.Cu") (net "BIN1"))
 (segment (start 104.934 44.286) (end 104.934 41.984) (width 0.2) (layer "F.Cu") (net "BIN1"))
 (segment (start 104.934 41.984) (end 107.236 41.984) (width 0.2) (layer "F.Cu") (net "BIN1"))
 (segment (start 102.4745 65.207408) (end 95.6925 58.425408) (width 0.2) (layer "F.Cu") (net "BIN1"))
 (segment (start 107.236 43.664) (end 107.824 43.076) (width 0.2) (layer "F.Cu") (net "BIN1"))
 (segment (start 95.6925 58.425408) (end 95.6925 55.2075) (width 0.2) (layer "F.Cu") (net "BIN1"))
 (segment (start 106.614 44.286) (end 104.934 44.286) (width 0.2) (layer "F.Cu") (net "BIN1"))
 (segment (start 102.4745 73.21025) (end 102.4745 65.207408) (width 0.2) (layer "F.Cu") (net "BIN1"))
 (segment (start 95.6925 55.2075) (end 106.614 44.286) (width 0.2) (layer "F.Cu") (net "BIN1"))
 (segment (start 105.0145 73.0855) (end 108.2 69.9) (width 0.2) (layer "F.Cu") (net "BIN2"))
 (segment (start 105.0145 73.21025) (end 105.0145 73.0855) (width 0.2) (layer "F.Cu") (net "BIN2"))
 (via (at 108.2 69.9) (size 0.6) (drill 0.3) (layers "F.Cu" "B.Cu") (capping no) (covering (front no) (back no))
  (plugging (front no) (back no)) (filling no) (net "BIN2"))
 (segment (start 122.571 55.529) (end 122.571 51.899) (width 0.2) (layer "B.Cu") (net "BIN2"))
 (segment (start 122.571 51.899) (end 129.09 45.38) (width 0.2) (layer "B.Cu") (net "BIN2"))
 (segment (start 108.2 69.9) (end 122.571 55.529) (width 0.2) (layer "B.Cu") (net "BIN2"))
 (segment (start 99.9345 73.21025) (end 99.9345 69.9955) (width 0.2) (layer "F.Cu") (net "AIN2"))
 (segment (start 99.9345 69.9955) (end 101.715 68.215) (width 0.2) (layer "F.Cu") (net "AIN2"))
 (segment (start 101.715 68.215) (end 101.73 68.2) (width 0.2) (layer "F.Cu") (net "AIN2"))
 (via (at 101.715 68.215) (size 0.6) (drill 0.3) (layers "F.Cu" "B.Cu") (capping no) (covering (front no) (back no))
  (plugging (front no) (back no)) (filling no) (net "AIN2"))
 (segment (start 113.63 59.42) (end 104.835 68.215) (width 0.2) (layer "B.Cu") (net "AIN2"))
 (segment (start 113.6975 54.73366) (end 112.749 53.78516) (width 0.2) (layer "B.Cu") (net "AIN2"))
 (segment (start 113.63 59.42) (end 113.6975 59.3525) (width 0.2) (layer "B.Cu") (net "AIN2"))
 (segment (start 113.6975 59.3525) (end 113.6975 54.73366) (width 0.2) (layer "B.Cu") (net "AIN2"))
 (segment (start 112.749 53.78516) (end 112.749 49.021) (width 0.2) (layer "B.Cu") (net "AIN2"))
 (segment (start 113.7 59.35) (end 113.63 59.42) (width 0.2) (layer "B.Cu") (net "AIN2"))
 (segment (start 112.749 49.021) (end 116.39 45.38) (width 0.2) (layer "B.Cu") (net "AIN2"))
 (segment (start 104.835 68.215) (end 101.715 68.215) (width 0.2) (layer "B.Cu") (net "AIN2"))
 (segment (start 116.53 72.38) (end 116.53 58.425692) (width 0.2) (layer "F.Cu") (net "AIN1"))
 (segment (start 97.3945 75.2145) (end 97.7 75.52) (width 0.2) (layer "F.Cu") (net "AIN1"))
 (segment (start 114.951 46.481) (end 113.85 45.38) (width 0.2) (layer "F.Cu") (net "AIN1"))
 (segment (start 113.39 75.52) (end 116.53 72.38) (width 0.2) (layer "F.Cu") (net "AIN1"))
 (segment (start 97.7 75.52) (end 113.39 75.52) (width 0.2) (layer "F.Cu") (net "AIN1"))
 (segment (start 116.53 58.425692) (end 114.951 56.846692) (width 0.2) (layer "F.Cu") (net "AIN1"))
 (segment (start 114.951 56.846692) (end 114.951 46.481) (width 0.2) (layer "F.Cu") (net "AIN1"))
 (segment (start 97.3945 73.21025) (end 97.3945 75.2145) (width 0.2) (layer "F.Cu") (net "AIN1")))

